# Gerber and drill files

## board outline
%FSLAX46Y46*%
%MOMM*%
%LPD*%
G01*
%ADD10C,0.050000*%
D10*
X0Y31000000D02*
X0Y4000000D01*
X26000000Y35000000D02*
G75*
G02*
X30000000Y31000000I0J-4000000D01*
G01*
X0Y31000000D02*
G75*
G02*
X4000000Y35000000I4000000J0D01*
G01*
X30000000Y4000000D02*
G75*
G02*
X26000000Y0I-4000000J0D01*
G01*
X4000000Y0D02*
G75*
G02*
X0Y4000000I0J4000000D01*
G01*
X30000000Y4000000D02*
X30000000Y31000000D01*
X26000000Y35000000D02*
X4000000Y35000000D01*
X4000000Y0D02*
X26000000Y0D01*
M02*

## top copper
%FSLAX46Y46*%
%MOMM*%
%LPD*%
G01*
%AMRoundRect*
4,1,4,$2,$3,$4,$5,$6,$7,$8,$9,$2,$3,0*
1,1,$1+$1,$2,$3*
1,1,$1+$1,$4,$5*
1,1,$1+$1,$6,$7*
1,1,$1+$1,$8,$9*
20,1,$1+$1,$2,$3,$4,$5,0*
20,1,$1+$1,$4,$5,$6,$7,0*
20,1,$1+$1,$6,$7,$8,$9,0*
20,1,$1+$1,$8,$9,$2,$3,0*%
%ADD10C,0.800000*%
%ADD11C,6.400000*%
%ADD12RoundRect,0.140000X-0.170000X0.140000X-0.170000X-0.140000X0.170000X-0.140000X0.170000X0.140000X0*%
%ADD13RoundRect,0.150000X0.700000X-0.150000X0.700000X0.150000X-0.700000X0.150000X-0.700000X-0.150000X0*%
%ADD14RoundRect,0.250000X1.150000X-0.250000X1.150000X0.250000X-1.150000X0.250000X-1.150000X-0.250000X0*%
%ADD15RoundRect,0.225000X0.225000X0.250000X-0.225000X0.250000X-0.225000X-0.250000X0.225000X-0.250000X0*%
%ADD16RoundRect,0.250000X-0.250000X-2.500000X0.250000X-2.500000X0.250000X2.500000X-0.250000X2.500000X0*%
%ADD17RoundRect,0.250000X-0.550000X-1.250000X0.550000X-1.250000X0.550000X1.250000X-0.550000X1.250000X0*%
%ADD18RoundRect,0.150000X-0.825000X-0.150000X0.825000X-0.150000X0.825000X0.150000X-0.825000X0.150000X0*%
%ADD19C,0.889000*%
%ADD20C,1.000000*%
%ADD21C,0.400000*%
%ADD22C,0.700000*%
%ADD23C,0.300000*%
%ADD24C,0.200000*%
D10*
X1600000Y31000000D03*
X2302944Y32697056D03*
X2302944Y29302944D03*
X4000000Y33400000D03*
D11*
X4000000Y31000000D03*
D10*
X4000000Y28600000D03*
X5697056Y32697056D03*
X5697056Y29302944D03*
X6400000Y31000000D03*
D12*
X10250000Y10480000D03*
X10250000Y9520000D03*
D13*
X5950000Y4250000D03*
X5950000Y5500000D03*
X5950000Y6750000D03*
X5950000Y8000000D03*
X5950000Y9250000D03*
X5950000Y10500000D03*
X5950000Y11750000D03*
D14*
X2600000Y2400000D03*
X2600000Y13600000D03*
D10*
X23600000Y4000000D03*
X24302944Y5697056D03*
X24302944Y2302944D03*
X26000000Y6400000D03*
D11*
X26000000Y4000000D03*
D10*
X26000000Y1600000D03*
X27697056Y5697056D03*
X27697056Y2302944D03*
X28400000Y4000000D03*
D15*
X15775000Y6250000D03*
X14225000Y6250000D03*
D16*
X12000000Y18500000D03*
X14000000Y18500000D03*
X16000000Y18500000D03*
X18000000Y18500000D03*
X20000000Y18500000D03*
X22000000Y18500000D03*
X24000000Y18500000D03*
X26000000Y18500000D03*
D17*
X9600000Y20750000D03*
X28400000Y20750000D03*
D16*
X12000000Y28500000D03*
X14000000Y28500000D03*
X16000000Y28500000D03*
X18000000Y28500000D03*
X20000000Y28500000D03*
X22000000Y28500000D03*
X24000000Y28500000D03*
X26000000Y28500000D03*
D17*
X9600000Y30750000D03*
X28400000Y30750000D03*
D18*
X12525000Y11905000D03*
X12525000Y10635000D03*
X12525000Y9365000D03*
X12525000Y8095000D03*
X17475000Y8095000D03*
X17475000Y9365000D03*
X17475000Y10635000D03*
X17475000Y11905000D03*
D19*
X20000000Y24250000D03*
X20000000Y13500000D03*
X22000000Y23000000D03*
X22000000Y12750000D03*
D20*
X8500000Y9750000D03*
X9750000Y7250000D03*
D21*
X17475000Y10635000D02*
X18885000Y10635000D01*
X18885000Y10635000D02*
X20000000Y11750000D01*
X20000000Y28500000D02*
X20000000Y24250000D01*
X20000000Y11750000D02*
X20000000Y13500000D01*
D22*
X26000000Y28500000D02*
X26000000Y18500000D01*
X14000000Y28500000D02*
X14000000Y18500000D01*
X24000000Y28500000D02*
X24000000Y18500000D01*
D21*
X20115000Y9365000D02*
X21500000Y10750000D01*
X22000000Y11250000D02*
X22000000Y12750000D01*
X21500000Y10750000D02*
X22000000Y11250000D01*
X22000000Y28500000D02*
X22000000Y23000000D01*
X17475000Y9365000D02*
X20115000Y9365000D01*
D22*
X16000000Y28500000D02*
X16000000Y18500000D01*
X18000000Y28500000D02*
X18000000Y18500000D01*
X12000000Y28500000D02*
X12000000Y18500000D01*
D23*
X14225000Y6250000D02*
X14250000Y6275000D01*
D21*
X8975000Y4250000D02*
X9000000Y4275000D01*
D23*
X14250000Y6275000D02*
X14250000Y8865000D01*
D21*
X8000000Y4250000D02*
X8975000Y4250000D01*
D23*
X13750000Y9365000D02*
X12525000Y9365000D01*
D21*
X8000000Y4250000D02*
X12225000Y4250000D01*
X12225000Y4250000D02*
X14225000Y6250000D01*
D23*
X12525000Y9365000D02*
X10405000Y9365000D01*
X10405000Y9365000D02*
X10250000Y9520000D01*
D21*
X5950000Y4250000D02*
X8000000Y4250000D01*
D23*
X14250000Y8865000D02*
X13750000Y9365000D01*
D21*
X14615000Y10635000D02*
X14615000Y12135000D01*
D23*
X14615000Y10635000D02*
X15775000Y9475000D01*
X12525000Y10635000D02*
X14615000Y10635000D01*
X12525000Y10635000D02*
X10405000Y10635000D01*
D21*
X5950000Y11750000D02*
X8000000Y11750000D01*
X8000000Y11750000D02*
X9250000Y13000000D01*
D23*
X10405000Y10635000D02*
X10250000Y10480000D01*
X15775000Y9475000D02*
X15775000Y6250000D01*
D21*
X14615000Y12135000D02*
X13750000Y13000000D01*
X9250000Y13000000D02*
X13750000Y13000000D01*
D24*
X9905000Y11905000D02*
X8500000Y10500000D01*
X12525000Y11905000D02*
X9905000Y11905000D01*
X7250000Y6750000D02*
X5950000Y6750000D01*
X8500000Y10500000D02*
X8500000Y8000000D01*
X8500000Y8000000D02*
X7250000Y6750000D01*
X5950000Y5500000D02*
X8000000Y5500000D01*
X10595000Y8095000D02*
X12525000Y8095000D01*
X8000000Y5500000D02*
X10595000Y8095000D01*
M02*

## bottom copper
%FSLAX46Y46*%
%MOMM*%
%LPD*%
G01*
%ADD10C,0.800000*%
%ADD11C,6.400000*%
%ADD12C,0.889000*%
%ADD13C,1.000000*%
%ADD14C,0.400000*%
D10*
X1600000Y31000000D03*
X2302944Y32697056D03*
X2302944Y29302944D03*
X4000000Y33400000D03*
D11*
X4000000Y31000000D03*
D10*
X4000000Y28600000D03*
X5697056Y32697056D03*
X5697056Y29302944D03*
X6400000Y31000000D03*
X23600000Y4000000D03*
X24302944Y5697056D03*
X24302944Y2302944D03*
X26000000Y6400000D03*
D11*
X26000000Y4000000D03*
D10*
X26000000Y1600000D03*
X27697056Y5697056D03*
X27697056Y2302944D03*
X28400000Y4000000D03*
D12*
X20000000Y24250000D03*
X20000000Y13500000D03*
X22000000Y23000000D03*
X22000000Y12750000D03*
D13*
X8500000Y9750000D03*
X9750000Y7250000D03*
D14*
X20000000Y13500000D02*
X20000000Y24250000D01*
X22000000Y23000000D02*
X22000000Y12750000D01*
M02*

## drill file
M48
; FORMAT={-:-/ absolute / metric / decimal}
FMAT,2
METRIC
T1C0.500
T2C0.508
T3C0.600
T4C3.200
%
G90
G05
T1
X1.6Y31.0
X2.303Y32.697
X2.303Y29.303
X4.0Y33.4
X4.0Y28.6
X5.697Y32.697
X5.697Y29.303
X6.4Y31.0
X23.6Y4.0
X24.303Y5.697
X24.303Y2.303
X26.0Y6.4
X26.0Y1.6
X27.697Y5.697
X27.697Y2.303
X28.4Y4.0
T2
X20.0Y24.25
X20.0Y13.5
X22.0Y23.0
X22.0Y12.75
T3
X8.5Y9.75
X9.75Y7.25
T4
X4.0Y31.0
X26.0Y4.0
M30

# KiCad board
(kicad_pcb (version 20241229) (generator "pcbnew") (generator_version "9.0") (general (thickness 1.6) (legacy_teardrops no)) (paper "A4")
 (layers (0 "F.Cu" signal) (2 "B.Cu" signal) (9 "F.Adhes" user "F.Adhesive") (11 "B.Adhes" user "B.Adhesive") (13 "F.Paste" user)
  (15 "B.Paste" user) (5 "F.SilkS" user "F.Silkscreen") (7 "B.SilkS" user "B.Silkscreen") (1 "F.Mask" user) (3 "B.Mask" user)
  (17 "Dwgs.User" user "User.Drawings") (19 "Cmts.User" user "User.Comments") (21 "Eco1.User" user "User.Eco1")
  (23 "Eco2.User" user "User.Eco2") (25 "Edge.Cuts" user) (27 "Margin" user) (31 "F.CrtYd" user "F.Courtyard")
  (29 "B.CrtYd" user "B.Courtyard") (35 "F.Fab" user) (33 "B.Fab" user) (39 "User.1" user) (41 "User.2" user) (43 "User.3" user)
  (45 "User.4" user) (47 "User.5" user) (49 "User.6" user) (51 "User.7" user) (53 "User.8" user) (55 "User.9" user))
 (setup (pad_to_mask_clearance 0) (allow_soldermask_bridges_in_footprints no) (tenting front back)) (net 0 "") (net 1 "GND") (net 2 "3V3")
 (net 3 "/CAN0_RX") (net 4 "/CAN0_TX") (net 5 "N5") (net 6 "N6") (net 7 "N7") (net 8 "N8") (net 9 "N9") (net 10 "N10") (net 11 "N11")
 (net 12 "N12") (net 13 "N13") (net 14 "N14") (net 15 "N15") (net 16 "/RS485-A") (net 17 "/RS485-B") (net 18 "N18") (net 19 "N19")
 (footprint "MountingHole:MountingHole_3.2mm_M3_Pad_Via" (layer "F.Cu") (at 4 -31)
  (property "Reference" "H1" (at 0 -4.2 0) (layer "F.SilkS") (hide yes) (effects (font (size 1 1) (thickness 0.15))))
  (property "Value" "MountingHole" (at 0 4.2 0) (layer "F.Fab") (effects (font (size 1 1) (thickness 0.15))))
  (pad "1" thru_hole circle (at -2.4 0) (size 0.8 0.8) (drill 0.5) (layers "*.Cu" "*.Mask") (remove_unused_layers no) (zone_connect 2))
  (pad "1" thru_hole circle (at -1.697056 -1.697056) (size 0.8 0.8) (drill 0.5) (layers "*.Cu" "*.Mask") (remove_unused_layers no)
   (zone_connect 2))
  (pad "1" thru_hole circle (at -1.697056 1.697056) (size 0.8 0.8) (drill 0.5) (layers "*.Cu" "*.Mask") (remove_unused_layers no)
   (zone_connect 2))
  (pad "1" thru_hole circle (at 0 -2.4) (size 0.8 0.8) (drill 0.5) (layers "*.Cu" "*.Mask") (remove_unused_layers no) (zone_connect 2))
  (pad "1" thru_hole circle (at 0 0) (size 6.4 6.4) (drill 3.2) (layers "*.Cu" "*.Mask") (remove_unused_layers no))
  (pad "1" thru_hole circle (at 0 2.4) (size 0.8 0.8) (drill 0.5) (layers "*.Cu" "*.Mask") (remove_unused_layers no) (zone_connect 2))
  (pad "1" thru_hole circle (at 1.697056 -1.697056) (size 0.8 0.8) (drill 0.5) (layers "*.Cu" "*.Mask") (remove_unused_layers no)
   (zone_connect 2))
  (pad "1" thru_hole circle (at 1.697056 1.697056) (size 0.8 0.8) (drill 0.5) (layers "*.Cu" "*.Mask") (remove_unused_layers no)
   (zone_connect 2))
  (pad "1" thru_hole circle (at 2.4 0) (size 0.8 0.8) (drill 0.5) (layers "*.Cu" "*.Mask") (remove_unused_layers no) (zone_connect 2)))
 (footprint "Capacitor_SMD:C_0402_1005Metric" (layer "F.Cu") (at 10.25 -10 -90)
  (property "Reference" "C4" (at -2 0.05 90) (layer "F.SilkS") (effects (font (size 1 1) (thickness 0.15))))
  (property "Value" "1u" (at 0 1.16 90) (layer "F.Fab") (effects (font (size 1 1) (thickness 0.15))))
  (pad "1" smd roundrect (at -0.48 0 270) (size 0.56 0.62) (layers "F.Cu" "F.Mask" "F.Paste") (roundrect_rratio 0.25) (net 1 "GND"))
  (pad "2" smd roundrect (at 0.48 0 270) (size 0.56 0.62) (layers "F.Cu" "F.Mask" "F.Paste") (roundrect_rratio 0.25) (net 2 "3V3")))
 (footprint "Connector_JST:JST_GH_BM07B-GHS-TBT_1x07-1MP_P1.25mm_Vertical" (layer "F.Cu") (at 4 -8 90)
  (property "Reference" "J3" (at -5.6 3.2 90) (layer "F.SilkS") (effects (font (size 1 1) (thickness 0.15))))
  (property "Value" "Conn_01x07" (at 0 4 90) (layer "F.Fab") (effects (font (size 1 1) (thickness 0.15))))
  (pad "1" smd roundrect (at -3.75 1.95 90) (size 0.6 1.7) (layers "F.Cu" "F.Mask" "F.Paste") (roundrect_rratio 0.25) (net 2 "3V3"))
  (pad "2" smd roundrect (at -2.5 1.95 90) (size 0.6 1.7) (layers "F.Cu" "F.Mask" "F.Paste") (roundrect_rratio 0.25) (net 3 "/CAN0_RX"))
  (pad "3" smd roundrect (at -1.25 1.95 90) (size 0.6 1.7) (layers "F.Cu" "F.Mask" "F.Paste") (roundrect_rratio 0.25) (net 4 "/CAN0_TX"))
  (pad "4" smd roundrect (at 0 1.95 90) (size 0.6 1.7) (layers "F.Cu" "F.Mask" "F.Paste") (roundrect_rratio 0.25) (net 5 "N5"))
  (pad "5" smd roundrect (at 1.25 1.95 90) (size 0.6 1.7) (layers "F.Cu" "F.Mask" "F.Paste") (roundrect_rratio 0.25) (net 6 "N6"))
  (pad "6" smd roundrect (at 2.5 1.95 90) (size 0.6 1.7) (layers "F.Cu" "F.Mask" "F.Paste") (roundrect_rratio 0.25) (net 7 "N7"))
  (pad "7" smd roundrect (at 3.75 1.95 90) (size 0.6 1.7) (layers "F.Cu" "F.Mask" "F.Paste") (roundrect_rratio 0.25) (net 1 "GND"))
  (pad "MP" smd roundrect (at -5.6 -1.4 90) (size 1 2.8) (layers "F.Cu" "F.Mask" "F.Paste") (roundrect_rratio 0.25))
  (pad "MP" smd roundrect (at 5.6 -1.4 90) (size 1 2.8) (layers "F.Cu" "F.Mask" "F.Paste") (roundrect_rratio 0.25)))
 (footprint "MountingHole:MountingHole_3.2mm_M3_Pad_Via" (layer "F.Cu") (at 26 -4)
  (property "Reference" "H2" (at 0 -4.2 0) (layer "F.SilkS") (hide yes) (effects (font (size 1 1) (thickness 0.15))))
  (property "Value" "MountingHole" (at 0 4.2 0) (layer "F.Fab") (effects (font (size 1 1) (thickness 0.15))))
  (pad "1" thru_hole circle (at -2.4 0) (size 0.8 0.8) (drill 0.5) (layers "*.Cu" "*.Mask") (remove_unused_layers no) (zone_connect 2))
  (pad "1" thru_hole circle (at -1.697056 -1.697056) (size 0.8 0.8) (drill 0.5) (layers "*.Cu" "*.Mask") (remove_unused_layers no)
   (zone_connect 2))
  (pad "1" thru_hole circle (at -1.697056 1.697056) (size 0.8 0.8) (drill 0.5) (layers "*.Cu" "*.Mask") (remove_unused_layers no)
   (zone_connect 2))
  (pad "1" thru_hole circle (at 0 -2.4) (size 0.8 0.8) (drill 0.5) (layers "*.Cu" "*.Mask") (remove_unused_layers no) (zone_connect 2))
  (pad "1" thru_hole circle (at 0 0) (size 6.4 6.4) (drill 3.2) (layers "*.Cu" "*.Mask") (remove_unused_layers no))
  (pad "1" thru_hole circle (at 0 2.4) (size 0.8 0.8) (drill 0.5) (layers "*.Cu" "*.Mask") (remove_unused_layers no) (zone_connect 2))
  (pad "1" thru_hole circle (at 1.697056 -1.697056) (size 0.8 0.8) (drill 0.5) (layers "*.Cu" "*.Mask") (remove_unused_layers no)
   (zone_connect 2))
  (pad "1" thru_hole circle (at 1.697056 1.697056) (size 0.8 0.8) (drill 0.5) (layers "*.Cu" "*.Mask") (remove_unused_layers no)
   (zone_connect 2))
  (pad "1" thru_hole circle (at 2.4 0) (size 0.8 0.8) (drill 0.5) (layers "*.Cu" "*.Mask") (remove_unused_layers no) (zone_connect 2)))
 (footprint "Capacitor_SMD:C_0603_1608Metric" (layer "F.Cu") (at 15 -6.25 180)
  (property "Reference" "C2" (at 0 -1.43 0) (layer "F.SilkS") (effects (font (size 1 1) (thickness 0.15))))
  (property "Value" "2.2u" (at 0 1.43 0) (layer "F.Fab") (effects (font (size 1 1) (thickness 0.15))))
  (pad "1" smd roundrect (at -0.775 0 180) (size 0.9 0.95) (layers "F.Cu" "F.Mask" "F.Paste") (roundrect_rratio 0.25) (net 1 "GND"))
  (pad "2" smd roundrect (at 0.775 0 180) (size 0.9 0.95) (layers "F.Cu" "F.Mask" "F.Paste") (roundrect_rratio 0.25) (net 2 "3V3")))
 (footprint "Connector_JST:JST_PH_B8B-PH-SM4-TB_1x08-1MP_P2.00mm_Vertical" (layer "F.Cu") (at 19 -19)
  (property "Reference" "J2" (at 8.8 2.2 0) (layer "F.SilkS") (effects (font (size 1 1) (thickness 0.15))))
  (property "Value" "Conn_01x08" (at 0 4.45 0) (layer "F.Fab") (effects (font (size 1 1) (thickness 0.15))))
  (pad "1" smd roundrect (at -7 0.5) (size 1 5.5) (layers "F.Cu" "F.Mask" "F.Paste") (roundrect_rratio 0.25) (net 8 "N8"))
  (pad "2" smd roundrect (at -5 0.5) (size 1 5.5) (layers "F.Cu" "F.Mask" "F.Paste") (roundrect_rratio 0.25) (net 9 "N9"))
  (pad "3" smd roundrect (at -3 0.5) (size 1 5.5) (layers "F.Cu" "F.Mask" "F.Paste") (roundrect_rratio 0.25) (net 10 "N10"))
  (pad "4" smd roundrect (at -1 0.5) (size 1 5.5) (layers "F.Cu" "F.Mask" "F.Paste") (roundrect_rratio 0.25) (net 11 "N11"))
  (pad "5" smd roundrect (at 1 0.5) (size 1 5.5) (layers "F.Cu" "F.Mask" "F.Paste") (roundrect_rratio 0.25) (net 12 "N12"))
  (pad "6" smd roundrect (at 3 0.5) (size 1 5.5) (layers "F.Cu" "F.Mask" "F.Paste") (roundrect_rratio 0.25) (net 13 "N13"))
  (pad "7" smd roundrect (at 5 0.5) (size 1 5.5) (layers "F.Cu" "F.Mask" "F.Paste") (roundrect_rratio 0.25) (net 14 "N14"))
  (pad "8" smd roundrect (at 7 0.5) (size 1 5.5) (layers "F.Cu" "F.Mask" "F.Paste") (roundrect_rratio 0.25) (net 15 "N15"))
  (pad "MP" smd roundrect (at -9.4 -1.75) (size 1.6 3) (layers "F.Cu" "F.Mask" "F.Paste") (roundrect_rratio 0.15625))
  (pad "MP" smd roundrect (at 9.4 -1.75) (size 1.6 3) (layers "F.Cu" "F.Mask" "F.Paste") (roundrect_rratio 0.15625)))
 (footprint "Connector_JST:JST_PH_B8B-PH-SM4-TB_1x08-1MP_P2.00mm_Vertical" (layer "F.Cu") (at 19 -29)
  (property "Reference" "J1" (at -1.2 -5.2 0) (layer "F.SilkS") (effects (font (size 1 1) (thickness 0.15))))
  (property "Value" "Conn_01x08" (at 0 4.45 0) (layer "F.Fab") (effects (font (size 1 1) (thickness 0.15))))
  (pad "1" smd roundrect (at -7 0.5) (size 1 5.5) (layers "F.Cu" "F.Mask" "F.Paste") (roundrect_rratio 0.25) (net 8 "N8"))
  (pad "2" smd roundrect (at -5 0.5) (size 1 5.5) (layers "F.Cu" "F.Mask" "F.Paste") (roundrect_rratio 0.25) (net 9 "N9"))
  (pad "3" smd roundrect (at -3 0.5) (size 1 5.5) (layers "F.Cu" "F.Mask" "F.Paste") (roundrect_rratio 0.25) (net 10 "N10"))
  (pad "4" smd roundrect (at -1 0.5) (size 1 5.5) (layers "F.Cu" "F.Mask" "F.Paste") (roundrect_rratio 0.25) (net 11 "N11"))
  (pad "5" smd roundrect (at 1 0.5) (size 1 5.5) (layers "F.Cu" "F.Mask" "F.Paste") (roundrect_rratio 0.25) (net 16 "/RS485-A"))
  (pad "6" smd roundrect (at 3 0.5) (size 1 5.5) (layers "F.Cu" "F.Mask" "F.Paste") (roundrect_rratio 0.25) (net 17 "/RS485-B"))
  (pad "7" smd roundrect (at 5 0.5) (size 1 5.5) (layers "F.Cu" "F.Mask" "F.Paste") (roundrect_rratio 0.25) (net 14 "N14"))
  (pad "8" smd roundrect (at 7 0.5) (size 1 5.5) (layers "F.Cu" "F.Mask" "F.Paste") (roundrect_rratio 0.25) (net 15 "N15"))
  (pad "MP" smd roundrect (at -9.4 -1.75) (size 1.6 3) (layers "F.Cu" "F.Mask" "F.Paste") (roundrect_rratio 0.15625))
  (pad "MP" smd roundrect (at 9.4 -1.75) (size 1.6 3) (layers "F.Cu" "F.Mask" "F.Paste") (roundrect_rratio 0.15625)))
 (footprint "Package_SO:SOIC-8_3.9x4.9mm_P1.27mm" (layer "F.Cu") (at 15 -10)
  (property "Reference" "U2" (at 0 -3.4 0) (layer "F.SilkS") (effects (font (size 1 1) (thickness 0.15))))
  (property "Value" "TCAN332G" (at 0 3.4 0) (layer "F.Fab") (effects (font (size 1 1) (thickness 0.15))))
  (pad "1" smd roundrect (at -2.475 -1.905) (size 1.95 0.6) (layers "F.Cu" "F.Mask" "F.Paste") (roundrect_rratio 0.25) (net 4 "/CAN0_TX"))
  (pad "2" smd roundrect (at -2.475 -0.635) (size 1.95 0.6) (layers "F.Cu" "F.Mask" "F.Paste") (roundrect_rratio 0.25) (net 1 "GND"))
  (pad "3" smd roundrect (at -2.475 0.635) (size 1.95 0.6) (layers "F.Cu" "F.Mask" "F.Paste") (roundrect_rratio 0.25) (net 2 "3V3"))
  (pad "4" smd roundrect (at -2.475 1.905) (size 1.95 0.6) (layers "F.Cu" "F.Mask" "F.Paste") (roundrect_rratio 0.25) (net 3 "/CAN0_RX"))
  (pad "5" smd roundrect (at 2.475 1.905) (size 1.95 0.6) (layers "F.Cu" "F.Mask" "F.Paste") (roundrect_rratio 0.25) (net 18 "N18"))
  (pad "6" smd roundrect (at 2.475 0.635) (size 1.95 0.6) (layers "F.Cu" "F.Mask" "F.Paste") (roundrect_rratio 0.25) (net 17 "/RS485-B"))
  (pad "7" smd roundrect (at 2.475 -0.635) (size 1.95 0.6) (layers "F.Cu" "F.Mask" "F.Paste") (roundrect_rratio 0.25) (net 16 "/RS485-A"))
  (pad "8" smd roundrect (at 2.475 -1.905) (size 1.95 0.6) (layers "F.Cu" "F.Mask" "F.Paste") (roundrect_rratio 0.25) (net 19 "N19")))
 (gr_line (start 0 -31) (end 0 -4) (stroke (width 0.05) (type default)) (layer "Edge.Cuts"))
 (gr_arc (start 26 -35) (mid 28.828427 -33.828427) (end 30 -31) (stroke (width 0.05) (type default)) (layer "Edge.Cuts"))
 (gr_arc (start 0 -31) (mid 1.171573 -33.828427) (end 4 -35) (stroke (width 0.05) (type default)) (layer "Edge.Cuts"))
 (gr_arc (start 30 -4) (mid 28.828427 -1.171573) (end 26 0) (stroke (width 0.05) (type default)) (layer "Edge.Cuts"))
 (gr_arc (start 4 0) (mid 1.171573 -1.171573) (end 0 -4) (stroke (width 0.05) (type default)) (layer "Edge.Cuts"))
 (gr_line (start 30 -4) (end 30 -31) (stroke (width 0.05) (type default)) (layer "Edge.Cuts"))
 (gr_line (start 26 -35) (end 4 -35) (stroke (width 0.05) (type default)) (layer "Edge.Cuts"))
 (gr_line (start 4 0) (end 26 0) (stroke (width 0.05) (type default)) (layer "Edge.Cuts"))
 (segment (start 17.475 -10.635) (end 18.885 -10.635) (width 0.4) (layer "F.Cu") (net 16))
 (segment (start 18.885 -10.635) (end 20 -11.75) (width 0.4) (layer "F.Cu") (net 16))
 (segment (start 20 -28.5) (end 20 -24.25) (width 0.4) (layer "F.Cu") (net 16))
 (segment (start 20 -11.75) (end 20 -13.5) (width 0.4) (layer "F.Cu") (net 16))
 (via (at 20 -24.25) (size 0.889) (drill 0.508) (layers "F.Cu" "B.Cu") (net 16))
 (via (at 20 -13.5) (size 0.889) (drill 0.508) (layers "F.Cu" "B.Cu") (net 16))
 (segment (start 20 -13.5) (end 20 -24.25) (width 0.4) (layer "B.Cu") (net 16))
 (segment (start 26 -28.5) (end 26 -18.5) (width 0.7) (layer "F.Cu") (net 15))
 (segment (start 14 -28.5) (end 14 -18.5) (width 0.7) (layer "F.Cu") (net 9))
 (segment (start 24 -28.5) (end 24 -18.5) (width 0.7) (layer "F.Cu") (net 14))
 (segment (start 20.115 -9.365) (end 21.5 -10.75) (width 0.4) (layer "F.Cu") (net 17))
 (segment (start 22 -11.25) (end 22 -12.75) (width 0.4) (layer "F.Cu") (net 17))
 (segment (start 21.5 -10.75) (end 22 -11.25) (width 0.4) (layer "F.Cu") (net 17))
 (segment (start 22 -28.5) (end 22 -23) (width 0.4) (layer "F.Cu") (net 17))
 (segment (start 17.475 -9.365) (end 20.115 -9.365) (width 0.4) (layer "F.Cu") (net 17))
 (via (at 22 -23) (size 0.889) (drill 0.508) (layers "F.Cu" "B.Cu") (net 17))
 (via (at 22 -12.75) (size 0.889) (drill 0.508) (layers "F.Cu" "B.Cu") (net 17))
 (segment (start 22 -23) (end 22 -12.75) (width 0.4) (layer "B.Cu") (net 17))
 (segment (start 16 -28.5) (end 16 -18.5) (width 0.7) (layer "F.Cu") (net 10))
 (segment (start 18 -28.5) (end 18 -18.5) (width 0.7) (layer "F.Cu") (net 11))
 (segment (start 12 -28.5) (end 12 -18.5) (width 0.7) (layer "F.Cu") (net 8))
 (segment (start 14.225 -6.25) (end 14.25 -6.275) (width 0.3) (layer "F.Cu") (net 2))
 (segment (start 8.975 -4.25) (end 9 -4.275) (width 0.4) (layer "F.Cu") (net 2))
 (segment (start 14.25 -6.275) (end 14.25 -8.865) (width 0.3) (layer "F.Cu") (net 2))
 (segment (start 8 -4.25) (end 8.975 -4.25) (width 0.4) (layer "F.Cu") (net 2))
 (segment (start 13.75 -9.365) (end 12.525 -9.365) (width 0.3) (layer "F.Cu") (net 2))
 (segment (start 8 -4.25) (end 12.225 -4.25) (width 0.4) (layer "F.Cu") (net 2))
 (segment (start 12.225 -4.25) (end 14.225 -6.25) (width 0.4) (layer "F.Cu") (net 2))
 (segment (start 12.525 -9.365) (end 10.405 -9.365) (width 0.3) (layer "F.Cu") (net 2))
 (segment (start 10.405 -9.365) (end 10.25 -9.52) (width 0.3) (layer "F.Cu") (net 2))
 (segment (start 5.95 -4.25) (end 8 -4.25) (width 0.4) (layer "F.Cu") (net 2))
 (segment (start 14.25 -8.865) (end 13.75 -9.365) (width 0.3) (layer "F.Cu") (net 2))
 (segment (start 14.615 -10.635) (end 14.615 -12.135) (width 0.4) (layer "F.Cu") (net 1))
 (segment (start 14.615 -10.635) (end 15.775 -9.475) (width 0.3) (layer "F.Cu") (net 1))
 (segment (start 12.525 -10.635) (end 14.615 -10.635) (width 0.3) (layer "F.Cu") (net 1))
 (segment (start 12.525 -10.635) (end 10.405 -10.635) (width 0.3) (layer "F.Cu") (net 1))
 (segment (start 5.95 -11.75) (end 8 -11.75) (width 0.4) (layer "F.Cu") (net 1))
 (segment (start 8 -11.75) (end 9.25 -13) (width 0.4) (layer "F.Cu") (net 1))
 (segment (start 10.405 -10.635) (end 10.25 -10.48) (width 0.3) (layer "F.Cu") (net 1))
 (segment (start 15.775 -9.475) (end 15.775 -6.25) (width 0.3) (layer "F.Cu") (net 1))
 (segment (start 14.615 -12.135) (end 13.75 -13) (width 0.4) (layer "F.Cu") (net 1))
 (segment (start 9.25 -13) (end 13.75 -13) (width 0.4) (layer "F.Cu") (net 1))
 (segment (start 9.905 -11.905) (end 8.5 -10.5) (width 0.2) (layer "F.Cu") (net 4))
 (segment (start 12.525 -11.905) (end 9.905 -11.905) (width 0.2) (layer "F.Cu") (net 4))
 (segment (start 7.25 -6.75) (end 5.95 -6.75) (width 0.2) (layer "F.Cu") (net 4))
 (segment (start 8.5 -10.5) (end 8.5 -8) (width 0.2) (layer "F.Cu") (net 4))
 (segment (start 8.5 -8) (end 7.25 -6.75) (width 0.2) (layer "F.Cu") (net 4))
 (via (at 8.5 -9.75) (size 1) (drill 0.6) (layers "F.Cu" "B.Cu") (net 4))
 (segment (start 5.95 -5.5) (end 8 -5.5) (width 0.2) (layer "F.Cu") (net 3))
 (segment (start 10.595 -8.095) (end 12.525 -8.095) (width 0.2) (layer "F.Cu") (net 3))
 (segment (start 8 -5.5) (end 10.595 -8.095) (width 0.2) (layer "F.Cu") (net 3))
 (via (at 9.75 -7.25) (size 1) (drill 0.6) (layers "F.Cu" "B.Cu") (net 3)))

